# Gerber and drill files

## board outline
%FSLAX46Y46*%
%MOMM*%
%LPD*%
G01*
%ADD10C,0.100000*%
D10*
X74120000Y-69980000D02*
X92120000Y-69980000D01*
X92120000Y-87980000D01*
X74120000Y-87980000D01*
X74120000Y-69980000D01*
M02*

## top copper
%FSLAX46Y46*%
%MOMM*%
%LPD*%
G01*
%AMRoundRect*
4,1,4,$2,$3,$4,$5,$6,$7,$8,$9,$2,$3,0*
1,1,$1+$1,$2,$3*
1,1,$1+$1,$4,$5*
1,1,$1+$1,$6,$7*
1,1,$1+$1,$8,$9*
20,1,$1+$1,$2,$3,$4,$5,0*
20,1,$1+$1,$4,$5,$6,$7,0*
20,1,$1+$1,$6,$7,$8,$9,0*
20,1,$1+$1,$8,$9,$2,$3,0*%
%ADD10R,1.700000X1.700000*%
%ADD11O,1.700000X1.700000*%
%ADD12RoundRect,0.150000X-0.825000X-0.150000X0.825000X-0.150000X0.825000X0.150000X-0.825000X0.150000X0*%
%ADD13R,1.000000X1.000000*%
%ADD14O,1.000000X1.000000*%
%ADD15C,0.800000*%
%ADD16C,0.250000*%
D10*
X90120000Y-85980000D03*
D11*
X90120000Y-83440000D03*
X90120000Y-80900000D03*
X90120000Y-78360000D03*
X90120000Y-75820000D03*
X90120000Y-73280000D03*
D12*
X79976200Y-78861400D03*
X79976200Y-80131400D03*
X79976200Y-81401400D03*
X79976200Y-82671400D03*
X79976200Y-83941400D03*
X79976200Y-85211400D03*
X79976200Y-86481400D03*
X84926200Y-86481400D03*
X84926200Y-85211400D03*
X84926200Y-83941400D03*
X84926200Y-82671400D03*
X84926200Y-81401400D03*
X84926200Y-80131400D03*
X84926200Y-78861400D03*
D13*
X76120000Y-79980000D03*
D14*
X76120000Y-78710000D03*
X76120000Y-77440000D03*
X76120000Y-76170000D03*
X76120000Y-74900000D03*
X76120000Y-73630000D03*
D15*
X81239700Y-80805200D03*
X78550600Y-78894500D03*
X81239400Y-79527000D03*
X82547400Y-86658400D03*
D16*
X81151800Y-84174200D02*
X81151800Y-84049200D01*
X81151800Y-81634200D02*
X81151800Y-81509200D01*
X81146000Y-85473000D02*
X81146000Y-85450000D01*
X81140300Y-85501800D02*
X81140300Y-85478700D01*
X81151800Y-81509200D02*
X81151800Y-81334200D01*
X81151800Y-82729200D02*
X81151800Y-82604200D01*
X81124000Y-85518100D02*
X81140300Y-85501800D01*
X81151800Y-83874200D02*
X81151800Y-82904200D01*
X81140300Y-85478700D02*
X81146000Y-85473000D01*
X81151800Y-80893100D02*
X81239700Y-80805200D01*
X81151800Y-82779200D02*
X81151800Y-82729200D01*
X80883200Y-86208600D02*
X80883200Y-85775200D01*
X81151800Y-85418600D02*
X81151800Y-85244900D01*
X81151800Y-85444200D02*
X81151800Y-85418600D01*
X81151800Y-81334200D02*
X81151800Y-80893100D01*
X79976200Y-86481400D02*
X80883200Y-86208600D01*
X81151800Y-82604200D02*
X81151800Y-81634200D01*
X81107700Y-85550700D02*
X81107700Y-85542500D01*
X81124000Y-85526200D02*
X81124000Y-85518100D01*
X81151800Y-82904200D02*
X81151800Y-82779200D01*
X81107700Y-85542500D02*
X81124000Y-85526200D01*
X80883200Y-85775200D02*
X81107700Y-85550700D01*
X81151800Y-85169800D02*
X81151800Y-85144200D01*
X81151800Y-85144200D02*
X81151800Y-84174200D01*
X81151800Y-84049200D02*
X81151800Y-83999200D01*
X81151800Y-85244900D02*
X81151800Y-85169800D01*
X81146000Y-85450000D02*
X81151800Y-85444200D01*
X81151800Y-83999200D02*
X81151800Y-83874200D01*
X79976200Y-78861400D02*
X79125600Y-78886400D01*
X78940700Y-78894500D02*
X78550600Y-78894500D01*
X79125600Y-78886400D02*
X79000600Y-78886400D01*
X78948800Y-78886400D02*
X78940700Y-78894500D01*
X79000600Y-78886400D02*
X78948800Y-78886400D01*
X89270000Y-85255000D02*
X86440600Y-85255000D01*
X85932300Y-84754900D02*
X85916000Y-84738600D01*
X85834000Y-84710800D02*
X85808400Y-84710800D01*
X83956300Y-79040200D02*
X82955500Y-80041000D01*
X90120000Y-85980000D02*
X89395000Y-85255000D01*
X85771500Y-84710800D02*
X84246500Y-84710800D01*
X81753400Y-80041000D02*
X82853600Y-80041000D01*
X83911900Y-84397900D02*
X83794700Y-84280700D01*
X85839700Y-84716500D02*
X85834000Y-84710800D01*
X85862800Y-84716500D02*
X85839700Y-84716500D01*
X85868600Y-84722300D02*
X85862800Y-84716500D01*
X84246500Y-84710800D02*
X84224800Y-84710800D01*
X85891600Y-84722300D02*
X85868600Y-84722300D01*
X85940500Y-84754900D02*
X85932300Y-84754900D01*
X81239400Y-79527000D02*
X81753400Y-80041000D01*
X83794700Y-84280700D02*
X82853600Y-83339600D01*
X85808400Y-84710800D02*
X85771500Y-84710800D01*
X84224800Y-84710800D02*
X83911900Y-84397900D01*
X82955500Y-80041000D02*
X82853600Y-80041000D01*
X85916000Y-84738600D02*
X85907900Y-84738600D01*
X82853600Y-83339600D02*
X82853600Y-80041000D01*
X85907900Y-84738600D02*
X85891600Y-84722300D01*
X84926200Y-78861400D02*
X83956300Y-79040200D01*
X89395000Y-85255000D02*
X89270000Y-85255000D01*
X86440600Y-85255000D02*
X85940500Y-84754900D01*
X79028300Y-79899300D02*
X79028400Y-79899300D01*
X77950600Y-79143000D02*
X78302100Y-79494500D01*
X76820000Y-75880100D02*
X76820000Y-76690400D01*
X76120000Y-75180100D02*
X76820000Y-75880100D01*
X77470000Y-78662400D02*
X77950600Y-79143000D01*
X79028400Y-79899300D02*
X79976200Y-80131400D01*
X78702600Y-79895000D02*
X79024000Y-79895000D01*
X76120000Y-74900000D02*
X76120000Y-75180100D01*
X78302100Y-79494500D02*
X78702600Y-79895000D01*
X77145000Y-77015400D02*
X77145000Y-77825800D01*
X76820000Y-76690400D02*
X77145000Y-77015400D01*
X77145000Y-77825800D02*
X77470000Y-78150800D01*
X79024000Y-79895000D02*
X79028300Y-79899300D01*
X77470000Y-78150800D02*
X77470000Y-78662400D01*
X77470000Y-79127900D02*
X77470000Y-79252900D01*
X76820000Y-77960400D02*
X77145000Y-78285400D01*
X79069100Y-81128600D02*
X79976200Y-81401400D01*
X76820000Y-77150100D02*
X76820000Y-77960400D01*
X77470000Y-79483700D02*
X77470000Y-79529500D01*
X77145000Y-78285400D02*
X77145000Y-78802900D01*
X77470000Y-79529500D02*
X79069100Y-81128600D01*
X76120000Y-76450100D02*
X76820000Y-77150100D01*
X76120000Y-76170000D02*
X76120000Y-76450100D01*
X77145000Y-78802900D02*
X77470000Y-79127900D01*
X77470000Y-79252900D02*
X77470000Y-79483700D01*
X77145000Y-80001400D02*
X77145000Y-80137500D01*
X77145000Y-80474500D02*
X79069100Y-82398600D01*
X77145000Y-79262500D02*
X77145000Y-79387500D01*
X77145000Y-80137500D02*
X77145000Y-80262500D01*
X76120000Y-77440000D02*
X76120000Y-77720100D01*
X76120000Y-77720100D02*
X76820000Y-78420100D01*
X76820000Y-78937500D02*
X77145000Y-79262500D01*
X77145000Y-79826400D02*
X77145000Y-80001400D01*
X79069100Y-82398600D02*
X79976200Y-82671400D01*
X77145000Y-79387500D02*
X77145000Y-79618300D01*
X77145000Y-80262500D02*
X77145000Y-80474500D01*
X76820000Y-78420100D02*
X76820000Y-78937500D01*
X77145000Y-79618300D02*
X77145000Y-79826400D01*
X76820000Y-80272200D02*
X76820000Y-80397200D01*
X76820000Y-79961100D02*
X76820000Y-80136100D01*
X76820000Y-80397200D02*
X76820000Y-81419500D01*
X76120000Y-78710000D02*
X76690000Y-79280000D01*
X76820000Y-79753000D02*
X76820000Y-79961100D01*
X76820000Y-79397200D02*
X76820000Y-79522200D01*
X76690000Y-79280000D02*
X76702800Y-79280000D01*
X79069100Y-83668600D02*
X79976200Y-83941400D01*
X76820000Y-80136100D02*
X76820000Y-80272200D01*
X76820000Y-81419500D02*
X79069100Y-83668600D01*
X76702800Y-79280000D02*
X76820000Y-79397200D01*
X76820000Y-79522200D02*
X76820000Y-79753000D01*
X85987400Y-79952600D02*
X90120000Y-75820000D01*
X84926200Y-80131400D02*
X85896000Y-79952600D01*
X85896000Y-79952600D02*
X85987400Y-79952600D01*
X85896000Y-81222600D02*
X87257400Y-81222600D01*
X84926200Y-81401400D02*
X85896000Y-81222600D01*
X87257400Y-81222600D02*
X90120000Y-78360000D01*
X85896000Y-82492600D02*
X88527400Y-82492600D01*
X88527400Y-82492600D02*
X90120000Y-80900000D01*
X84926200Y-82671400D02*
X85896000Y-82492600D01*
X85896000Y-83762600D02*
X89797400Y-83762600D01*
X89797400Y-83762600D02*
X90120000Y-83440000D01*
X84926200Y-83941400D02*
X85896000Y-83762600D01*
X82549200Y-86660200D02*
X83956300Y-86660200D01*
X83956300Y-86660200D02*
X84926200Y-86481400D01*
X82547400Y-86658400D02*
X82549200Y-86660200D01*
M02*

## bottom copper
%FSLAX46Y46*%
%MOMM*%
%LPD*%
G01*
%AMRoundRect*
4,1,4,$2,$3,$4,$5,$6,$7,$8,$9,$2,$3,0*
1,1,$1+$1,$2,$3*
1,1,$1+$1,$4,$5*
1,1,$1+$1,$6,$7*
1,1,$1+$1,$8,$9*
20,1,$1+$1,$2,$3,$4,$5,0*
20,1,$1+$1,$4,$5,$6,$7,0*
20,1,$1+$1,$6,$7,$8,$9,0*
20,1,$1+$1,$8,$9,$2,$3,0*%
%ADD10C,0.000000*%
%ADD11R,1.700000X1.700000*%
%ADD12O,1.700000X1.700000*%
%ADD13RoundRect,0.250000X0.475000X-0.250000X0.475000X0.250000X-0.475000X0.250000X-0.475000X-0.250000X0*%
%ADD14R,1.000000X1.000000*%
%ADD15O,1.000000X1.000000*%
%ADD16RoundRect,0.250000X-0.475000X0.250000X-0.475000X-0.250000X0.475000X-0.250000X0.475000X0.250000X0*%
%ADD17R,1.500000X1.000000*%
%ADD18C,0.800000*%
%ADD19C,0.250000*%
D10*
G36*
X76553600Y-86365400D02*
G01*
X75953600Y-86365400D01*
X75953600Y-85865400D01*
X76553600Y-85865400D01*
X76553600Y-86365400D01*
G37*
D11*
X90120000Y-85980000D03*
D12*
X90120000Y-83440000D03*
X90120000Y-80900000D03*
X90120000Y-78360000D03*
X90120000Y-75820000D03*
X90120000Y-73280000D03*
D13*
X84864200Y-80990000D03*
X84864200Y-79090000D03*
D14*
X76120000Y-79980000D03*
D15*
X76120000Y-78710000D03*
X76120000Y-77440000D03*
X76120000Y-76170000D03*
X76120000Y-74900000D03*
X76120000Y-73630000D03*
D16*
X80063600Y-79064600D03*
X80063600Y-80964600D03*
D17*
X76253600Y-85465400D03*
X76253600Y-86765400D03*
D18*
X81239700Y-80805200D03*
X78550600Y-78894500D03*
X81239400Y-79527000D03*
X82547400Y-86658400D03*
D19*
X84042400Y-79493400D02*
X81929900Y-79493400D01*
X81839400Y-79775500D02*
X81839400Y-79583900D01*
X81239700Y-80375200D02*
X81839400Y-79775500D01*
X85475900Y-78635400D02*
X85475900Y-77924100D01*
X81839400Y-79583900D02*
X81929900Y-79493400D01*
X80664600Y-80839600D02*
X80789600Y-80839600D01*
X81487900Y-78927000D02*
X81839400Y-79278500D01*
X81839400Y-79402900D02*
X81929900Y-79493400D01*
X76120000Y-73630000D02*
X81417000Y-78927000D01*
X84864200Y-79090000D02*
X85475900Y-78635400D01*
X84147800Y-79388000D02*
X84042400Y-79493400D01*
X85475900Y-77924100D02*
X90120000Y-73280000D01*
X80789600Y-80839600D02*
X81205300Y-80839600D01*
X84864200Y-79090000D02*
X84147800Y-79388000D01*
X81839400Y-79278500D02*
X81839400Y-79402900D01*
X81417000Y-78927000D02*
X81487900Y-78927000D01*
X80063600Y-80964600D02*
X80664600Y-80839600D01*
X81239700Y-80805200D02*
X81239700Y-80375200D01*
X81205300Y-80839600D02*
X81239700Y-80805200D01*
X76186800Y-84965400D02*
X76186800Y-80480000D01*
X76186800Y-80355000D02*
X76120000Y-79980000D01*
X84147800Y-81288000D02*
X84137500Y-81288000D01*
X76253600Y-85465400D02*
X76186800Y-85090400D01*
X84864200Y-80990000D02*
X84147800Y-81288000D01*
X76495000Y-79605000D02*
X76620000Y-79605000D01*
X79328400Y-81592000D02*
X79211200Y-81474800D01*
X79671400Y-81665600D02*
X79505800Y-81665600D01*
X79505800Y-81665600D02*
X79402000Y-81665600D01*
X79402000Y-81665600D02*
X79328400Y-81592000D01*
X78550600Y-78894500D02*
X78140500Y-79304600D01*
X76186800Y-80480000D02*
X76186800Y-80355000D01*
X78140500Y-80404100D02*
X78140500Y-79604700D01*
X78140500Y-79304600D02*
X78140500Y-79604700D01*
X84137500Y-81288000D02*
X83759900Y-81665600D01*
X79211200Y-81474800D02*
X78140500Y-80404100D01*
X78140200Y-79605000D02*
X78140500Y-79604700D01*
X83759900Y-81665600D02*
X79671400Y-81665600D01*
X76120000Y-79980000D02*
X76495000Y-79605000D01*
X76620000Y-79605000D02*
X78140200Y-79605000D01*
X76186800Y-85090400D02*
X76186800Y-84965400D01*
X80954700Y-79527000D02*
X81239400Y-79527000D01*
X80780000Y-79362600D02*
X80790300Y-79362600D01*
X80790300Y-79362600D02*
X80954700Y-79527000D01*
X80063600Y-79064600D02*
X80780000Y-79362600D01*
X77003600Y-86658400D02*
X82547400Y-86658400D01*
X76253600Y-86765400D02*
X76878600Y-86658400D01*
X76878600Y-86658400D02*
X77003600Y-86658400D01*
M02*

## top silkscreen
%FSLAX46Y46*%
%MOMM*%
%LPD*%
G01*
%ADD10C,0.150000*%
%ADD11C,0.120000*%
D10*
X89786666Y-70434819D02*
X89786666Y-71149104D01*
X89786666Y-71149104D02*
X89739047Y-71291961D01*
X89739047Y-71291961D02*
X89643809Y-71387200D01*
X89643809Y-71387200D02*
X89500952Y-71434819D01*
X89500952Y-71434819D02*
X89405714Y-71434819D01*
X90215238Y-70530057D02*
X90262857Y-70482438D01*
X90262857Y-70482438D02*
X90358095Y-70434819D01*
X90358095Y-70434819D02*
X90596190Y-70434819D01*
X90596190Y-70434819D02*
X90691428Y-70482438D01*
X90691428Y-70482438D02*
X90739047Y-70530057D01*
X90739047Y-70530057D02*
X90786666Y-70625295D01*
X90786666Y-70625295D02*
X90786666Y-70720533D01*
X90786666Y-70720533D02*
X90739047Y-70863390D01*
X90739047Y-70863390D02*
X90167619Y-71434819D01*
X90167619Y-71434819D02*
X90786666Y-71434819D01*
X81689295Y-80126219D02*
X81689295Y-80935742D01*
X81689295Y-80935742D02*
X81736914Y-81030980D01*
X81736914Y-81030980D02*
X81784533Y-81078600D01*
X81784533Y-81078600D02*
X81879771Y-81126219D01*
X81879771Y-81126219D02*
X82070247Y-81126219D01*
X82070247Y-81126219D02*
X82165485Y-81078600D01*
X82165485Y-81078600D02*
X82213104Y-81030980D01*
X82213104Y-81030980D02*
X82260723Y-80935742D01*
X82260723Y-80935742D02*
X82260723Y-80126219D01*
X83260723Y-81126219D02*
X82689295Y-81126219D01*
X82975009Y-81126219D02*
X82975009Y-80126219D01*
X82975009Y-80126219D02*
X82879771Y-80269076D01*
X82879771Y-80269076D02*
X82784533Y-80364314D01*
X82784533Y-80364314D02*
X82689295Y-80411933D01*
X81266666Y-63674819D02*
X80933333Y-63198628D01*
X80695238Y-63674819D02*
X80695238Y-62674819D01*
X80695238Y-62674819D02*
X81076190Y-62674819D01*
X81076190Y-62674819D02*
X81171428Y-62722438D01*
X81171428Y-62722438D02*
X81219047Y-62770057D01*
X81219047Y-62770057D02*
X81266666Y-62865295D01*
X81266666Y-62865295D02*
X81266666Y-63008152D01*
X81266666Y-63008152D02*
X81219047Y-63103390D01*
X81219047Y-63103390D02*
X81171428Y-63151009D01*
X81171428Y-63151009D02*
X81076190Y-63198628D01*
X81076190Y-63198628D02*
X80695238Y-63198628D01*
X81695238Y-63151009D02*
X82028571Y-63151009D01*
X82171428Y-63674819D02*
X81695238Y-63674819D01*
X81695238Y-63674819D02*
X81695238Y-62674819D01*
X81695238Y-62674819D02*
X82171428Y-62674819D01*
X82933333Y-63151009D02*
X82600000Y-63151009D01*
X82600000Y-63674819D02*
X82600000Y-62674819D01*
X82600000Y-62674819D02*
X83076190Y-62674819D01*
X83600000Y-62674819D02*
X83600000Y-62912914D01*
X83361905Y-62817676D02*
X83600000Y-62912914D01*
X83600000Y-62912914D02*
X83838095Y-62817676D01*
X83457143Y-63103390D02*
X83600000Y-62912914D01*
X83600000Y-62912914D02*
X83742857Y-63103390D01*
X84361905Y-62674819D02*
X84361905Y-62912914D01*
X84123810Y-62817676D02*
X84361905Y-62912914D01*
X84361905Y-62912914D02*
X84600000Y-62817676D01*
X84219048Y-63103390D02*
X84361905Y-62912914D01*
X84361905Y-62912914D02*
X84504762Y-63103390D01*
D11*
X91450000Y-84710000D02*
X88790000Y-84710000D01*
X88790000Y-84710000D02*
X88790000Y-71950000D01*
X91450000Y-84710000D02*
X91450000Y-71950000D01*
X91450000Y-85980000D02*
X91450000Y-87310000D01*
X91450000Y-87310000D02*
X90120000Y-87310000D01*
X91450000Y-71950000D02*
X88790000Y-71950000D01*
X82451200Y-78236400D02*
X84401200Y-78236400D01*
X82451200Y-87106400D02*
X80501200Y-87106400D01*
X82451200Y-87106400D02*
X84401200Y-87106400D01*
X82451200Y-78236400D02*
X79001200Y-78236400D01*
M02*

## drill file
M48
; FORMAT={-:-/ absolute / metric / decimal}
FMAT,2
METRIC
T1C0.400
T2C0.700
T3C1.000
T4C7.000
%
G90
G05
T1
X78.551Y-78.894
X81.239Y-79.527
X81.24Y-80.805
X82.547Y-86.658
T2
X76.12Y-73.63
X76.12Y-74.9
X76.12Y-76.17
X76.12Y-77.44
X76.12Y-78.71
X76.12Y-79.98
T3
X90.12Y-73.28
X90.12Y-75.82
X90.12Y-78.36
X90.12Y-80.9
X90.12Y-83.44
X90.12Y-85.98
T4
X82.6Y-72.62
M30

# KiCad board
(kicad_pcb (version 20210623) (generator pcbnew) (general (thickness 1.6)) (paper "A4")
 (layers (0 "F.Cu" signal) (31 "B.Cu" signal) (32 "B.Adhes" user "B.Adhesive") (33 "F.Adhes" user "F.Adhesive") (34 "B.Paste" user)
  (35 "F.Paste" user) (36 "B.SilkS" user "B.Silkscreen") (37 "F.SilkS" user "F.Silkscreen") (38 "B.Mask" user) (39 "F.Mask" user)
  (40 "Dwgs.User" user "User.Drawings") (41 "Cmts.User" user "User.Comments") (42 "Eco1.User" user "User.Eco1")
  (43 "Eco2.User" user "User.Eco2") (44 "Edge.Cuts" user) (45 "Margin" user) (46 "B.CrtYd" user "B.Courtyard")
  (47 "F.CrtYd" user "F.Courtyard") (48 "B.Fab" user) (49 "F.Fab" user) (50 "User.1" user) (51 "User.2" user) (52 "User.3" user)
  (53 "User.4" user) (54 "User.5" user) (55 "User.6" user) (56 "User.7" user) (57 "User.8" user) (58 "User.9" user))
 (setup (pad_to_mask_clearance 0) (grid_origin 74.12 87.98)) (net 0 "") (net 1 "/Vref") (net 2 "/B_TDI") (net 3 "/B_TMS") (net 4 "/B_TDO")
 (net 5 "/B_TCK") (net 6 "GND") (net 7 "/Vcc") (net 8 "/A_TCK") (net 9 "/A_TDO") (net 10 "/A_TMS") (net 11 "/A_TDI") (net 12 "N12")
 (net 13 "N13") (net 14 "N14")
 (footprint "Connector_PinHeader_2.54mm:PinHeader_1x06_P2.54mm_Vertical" (layer "F.Cu") (at 90.12 85.98 180)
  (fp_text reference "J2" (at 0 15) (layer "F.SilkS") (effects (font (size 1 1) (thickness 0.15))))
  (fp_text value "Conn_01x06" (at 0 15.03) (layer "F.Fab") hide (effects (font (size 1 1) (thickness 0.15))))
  (fp_line (start -1.33 1.27) (end 1.33 1.27) (layer "F.SilkS") (width 0.12))
  (fp_line (start 1.33 1.27) (end 1.33 14.03) (layer "F.SilkS") (width 0.12))
  (fp_line (start -1.33 1.27) (end -1.33 14.03) (layer "F.SilkS") (width 0.12))
  (fp_line (start -1.33 0) (end -1.33 -1.33) (layer "F.SilkS") (width 0.12))
  (fp_line (start -1.33 -1.33) (end 0 -1.33) (layer "F.SilkS") (width 0.12))
  (fp_line (start -1.33 14.03) (end 1.33 14.03) (layer "F.SilkS") (width 0.12))
  (pad "1" thru_hole rect locked (at 0 0 180) (size 1.7 1.7) (drill 1) (layers *.Cu *.Mask) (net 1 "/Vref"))
  (pad "2" thru_hole oval locked (at 0 2.54 180) (size 1.7 1.7) (drill 1) (layers *.Cu *.Mask) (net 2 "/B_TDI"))
  (pad "3" thru_hole oval locked (at 0 5.08 180) (size 1.7 1.7) (drill 1) (layers *.Cu *.Mask) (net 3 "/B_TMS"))
  (pad "4" thru_hole oval locked (at 0 7.62 180) (size 1.7 1.7) (drill 1) (layers *.Cu *.Mask) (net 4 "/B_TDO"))
  (pad "5" thru_hole oval locked (at 0 10.16 180) (size 1.7 1.7) (drill 1) (layers *.Cu *.Mask) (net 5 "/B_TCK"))
  (pad "6" thru_hole oval locked (at 0 12.7 180) (size 1.7 1.7) (drill 1) (layers *.Cu *.Mask) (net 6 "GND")))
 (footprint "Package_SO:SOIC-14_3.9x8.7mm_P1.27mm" (layer "F.Cu") (at 82.4512 82.6714)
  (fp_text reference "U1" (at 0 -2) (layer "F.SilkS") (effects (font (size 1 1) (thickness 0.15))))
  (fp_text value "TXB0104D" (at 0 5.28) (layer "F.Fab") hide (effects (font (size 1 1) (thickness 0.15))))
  (fp_line (start 0 -4.435) (end 1.95 -4.435) (layer "F.SilkS") (width 0.12))
  (fp_line (start 0 4.435) (end -1.95 4.435) (layer "F.SilkS") (width 0.12))
  (fp_line (start 0 4.435) (end 1.95 4.435) (layer "F.SilkS") (width 0.12))
  (fp_line (start 0 -4.435) (end -3.45 -4.435) (layer "F.SilkS") (width 0.12))
  (pad "1" smd roundrect locked (at -2.475 -3.81) (size 1.95 0.6) (layers "F.Cu" "F.Paste" "F.Mask") (roundrect_rratio 0.25) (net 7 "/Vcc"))
  (pad "2" smd roundrect locked (at -2.475 -2.54) (size 1.95 0.6) (layers "F.Cu" "F.Paste" "F.Mask") (roundrect_rratio 0.25)
   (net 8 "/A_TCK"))
  (pad "3" smd roundrect locked (at -2.475 -1.27) (size 1.95 0.6) (layers "F.Cu" "F.Paste" "F.Mask") (roundrect_rratio 0.25)
   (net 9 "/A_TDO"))
  (pad "4" smd roundrect locked (at -2.475 0) (size 1.95 0.6) (layers "F.Cu" "F.Paste" "F.Mask") (roundrect_rratio 0.25) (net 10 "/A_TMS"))
  (pad "5" smd roundrect locked (at -2.475 1.27) (size 1.95 0.6) (layers "F.Cu" "F.Paste" "F.Mask") (roundrect_rratio 0.25)
   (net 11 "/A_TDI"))
  (pad "6" smd roundrect locked (at -2.475 2.54) (size 1.95 0.6) (layers "F.Cu" "F.Paste" "F.Mask") (roundrect_rratio 0.25) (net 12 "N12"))
  (pad "7" smd roundrect locked (at -2.475 3.81) (size 1.95 0.6) (layers "F.Cu" "F.Paste" "F.Mask") (roundrect_rratio 0.25) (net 6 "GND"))
  (pad "8" smd roundrect locked (at 2.475 3.81) (size 1.95 0.6) (layers "F.Cu" "F.Paste" "F.Mask") (roundrect_rratio 0.25) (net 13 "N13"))
  (pad "9" smd roundrect locked (at 2.475 2.54) (size 1.95 0.6) (layers "F.Cu" "F.Paste" "F.Mask") (roundrect_rratio 0.25) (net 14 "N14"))
  (pad "10" smd roundrect locked (at 2.475 1.27) (size 1.95 0.6) (layers "F.Cu" "F.Paste" "F.Mask") (roundrect_rratio 0.25) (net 2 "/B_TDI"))
  (pad "11" smd roundrect locked (at 2.475 0) (size 1.95 0.6) (layers "F.Cu" "F.Paste" "F.Mask") (roundrect_rratio 0.25) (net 3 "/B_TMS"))
  (pad "12" smd roundrect locked (at 2.475 -1.27) (size 1.95 0.6) (layers "F.Cu" "F.Paste" "F.Mask") (roundrect_rratio 0.25)
   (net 4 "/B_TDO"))
  (pad "13" smd roundrect locked (at 2.475 -2.54) (size 1.95 0.6) (layers "F.Cu" "F.Paste" "F.Mask") (roundrect_rratio 0.25)
   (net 5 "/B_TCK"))
  (pad "14" smd roundrect locked (at 2.475 -3.81) (size 1.95 0.6) (layers "F.Cu" "F.Paste" "F.Mask") (roundrect_rratio 0.25) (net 1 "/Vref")))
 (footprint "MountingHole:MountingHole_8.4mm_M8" (layer "F.Cu") (at 82.6 72.62)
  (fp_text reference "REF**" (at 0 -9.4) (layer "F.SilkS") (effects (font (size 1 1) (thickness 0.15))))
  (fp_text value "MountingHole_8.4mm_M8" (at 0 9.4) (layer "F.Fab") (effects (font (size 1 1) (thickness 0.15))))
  (pad "" np_thru_hole circle (at 0 0) (size 7 7) (drill 7) (layers F&B.Cu *.Mask)))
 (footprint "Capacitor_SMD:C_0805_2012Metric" (layer "B.Cu") (at 84.8642 80.04 90)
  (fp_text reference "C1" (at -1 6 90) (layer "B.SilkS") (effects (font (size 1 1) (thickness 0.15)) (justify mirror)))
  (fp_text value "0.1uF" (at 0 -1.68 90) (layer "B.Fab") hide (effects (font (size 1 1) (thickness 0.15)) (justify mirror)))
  (pad "1" smd roundrect locked (at -0.95 0 90) (size 1 1.45) (layers "B.Cu" "B.Paste" "B.Mask") (roundrect_rratio 0.25) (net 7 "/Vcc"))
  (pad "2" smd roundrect locked (at 0.95 0 90) (size 1 1.45) (layers "B.Cu" "B.Paste" "B.Mask") (roundrect_rratio 0.25) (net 6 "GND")))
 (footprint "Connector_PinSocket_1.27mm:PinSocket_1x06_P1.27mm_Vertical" (layer "B.Cu") (at 76.12 79.98)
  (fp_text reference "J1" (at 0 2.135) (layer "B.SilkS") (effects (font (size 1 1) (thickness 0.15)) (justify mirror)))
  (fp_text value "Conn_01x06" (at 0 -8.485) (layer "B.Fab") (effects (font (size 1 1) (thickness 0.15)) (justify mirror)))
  (pad "1" thru_hole rect locked (at 0 0) (size 1 1) (drill 0.7) (layers *.Cu *.Mask) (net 7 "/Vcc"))
  (pad "2" thru_hole oval locked (at 0 -1.27) (size 1 1) (drill 0.7) (layers *.Cu *.Mask) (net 11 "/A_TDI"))
  (pad "3" thru_hole oval locked (at 0 -2.54) (size 1 1) (drill 0.7) (layers *.Cu *.Mask) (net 10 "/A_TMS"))
  (pad "4" thru_hole oval locked (at 0 -3.81) (size 1 1) (drill 0.7) (layers *.Cu *.Mask) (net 9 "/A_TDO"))
  (pad "5" thru_hole oval locked (at 0 -5.08) (size 1 1) (drill 0.7) (layers *.Cu *.Mask) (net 8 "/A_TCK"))
  (pad "6" thru_hole oval locked (at 0 -6.35) (size 1 1) (drill 0.7) (layers *.Cu *.Mask) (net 6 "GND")))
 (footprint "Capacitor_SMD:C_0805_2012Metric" (layer "B.Cu") (at 80.0636 80.0146 -90)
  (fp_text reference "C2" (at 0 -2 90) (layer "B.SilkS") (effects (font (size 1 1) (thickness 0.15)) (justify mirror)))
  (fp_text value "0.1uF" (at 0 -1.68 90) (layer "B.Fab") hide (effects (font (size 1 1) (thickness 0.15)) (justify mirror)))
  (pad "1" smd roundrect locked (at -0.95 0 270) (size 1 1.45) (layers "B.Cu" "B.Paste" "B.Mask") (roundrect_rratio 0.25) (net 1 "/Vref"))
  (pad "2" smd roundrect locked (at 0.95 0 270) (size 1 1.45) (layers "B.Cu" "B.Paste" "B.Mask") (roundrect_rratio 0.25) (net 6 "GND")))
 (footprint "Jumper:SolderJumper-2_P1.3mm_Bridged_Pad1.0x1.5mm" (layer "B.Cu") (at 76.2536 86.1154 -90)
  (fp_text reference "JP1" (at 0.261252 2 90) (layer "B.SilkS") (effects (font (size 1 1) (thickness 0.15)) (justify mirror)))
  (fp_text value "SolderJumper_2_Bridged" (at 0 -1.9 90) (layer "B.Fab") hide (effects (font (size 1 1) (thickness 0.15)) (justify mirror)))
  (fp_poly (pts (xy -0.25 0.3) (xy 0.25 0.3) (xy 0.25 -0.3) (xy -0.25 -0.3)) (layer "B.Cu") (width 0) (fill solid))
  (pad "1" smd rect locked (at -0.65 0 270) (size 1 1.5) (layers "B.Cu" "B.Mask") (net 7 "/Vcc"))
  (pad "2" smd rect locked (at 0.65 0 270) (size 1 1.5) (layers "B.Cu" "B.Mask") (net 13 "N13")))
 (gr_rect (start 92.12 87.98) (end 74.12 69.98) (layer "Edge.Cuts") (width 0.1) (fill none))
 (segment (start 81.1518 84.1742) (end 81.1518 84.0492) (width 0.25) (layer "F.Cu") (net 6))
 (segment (start 81.1518 81.6342) (end 81.1518 81.5092) (width 0.25) (layer "F.Cu") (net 6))
 (segment (start 81.146 85.473) (end 81.146 85.45) (width 0.25) (layer "F.Cu") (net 6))
 (segment (start 81.1403 85.5018) (end 81.1403 85.4787) (width 0.25) (layer "F.Cu") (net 6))
 (segment (start 81.1518 81.5092) (end 81.1518 81.3342) (width 0.25) (layer "F.Cu") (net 6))
 (segment (start 81.1518 82.7292) (end 81.1518 82.6042) (width 0.25) (layer "F.Cu") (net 6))
 (segment (start 81.124 85.5181) (end 81.1403 85.5018) (width 0.25) (layer "F.Cu") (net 6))
 (segment (start 81.1518 83.8742) (end 81.1518 82.9042) (width 0.25) (layer "F.Cu") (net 6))
 (segment (start 81.1403 85.4787) (end 81.146 85.473) (width 0.25) (layer "F.Cu") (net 6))
 (segment (start 81.1518 80.8931) (end 81.2397 80.8052) (width 0.25) (layer "F.Cu") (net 6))
 (segment (start 81.1518 82.7792) (end 81.1518 82.7292) (width 0.25) (layer "F.Cu") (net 6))
 (segment (start 80.8832 86.2086) (end 80.8832 85.7752) (width 0.25) (layer "F.Cu") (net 6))
 (segment (start 81.1518 85.4186) (end 81.1518 85.2449) (width 0.25) (layer "F.Cu") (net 6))
 (segment (start 81.1518 85.4442) (end 81.1518 85.4186) (width 0.25) (layer "F.Cu") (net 6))
 (segment (start 81.1518 81.3342) (end 81.1518 80.8931) (width 0.25) (layer "F.Cu") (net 6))
 (segment (start 79.9762 86.4814) (end 80.8832 86.2086) (width 0.25) (layer "F.Cu") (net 6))
 (segment (start 81.1518 82.6042) (end 81.1518 81.6342) (width 0.25) (layer "F.Cu") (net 6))
 (segment (start 81.1077 85.5507) (end 81.1077 85.5425) (width 0.25) (layer "F.Cu") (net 6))
 (segment (start 81.124 85.5262) (end 81.124 85.5181) (width 0.25) (layer "F.Cu") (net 6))
 (segment (start 81.1518 82.9042) (end 81.1518 82.7792) (width 0.25) (layer "F.Cu") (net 6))
 (segment (start 81.1077 85.5425) (end 81.124 85.5262) (width 0.25) (layer "F.Cu") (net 6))
 (segment (start 80.8832 85.7752) (end 81.1077 85.5507) (width 0.25) (layer "F.Cu") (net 6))
 (segment (start 81.1518 85.1698) (end 81.1518 85.1442) (width 0.25) (layer "F.Cu") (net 6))
 (segment (start 81.1518 85.1442) (end 81.1518 84.1742) (width 0.25) (layer "F.Cu") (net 6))
 (segment (start 81.1518 84.0492) (end 81.1518 83.9992) (width 0.25) (layer "F.Cu") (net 6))
 (segment (start 81.1518 85.2449) (end 81.1518 85.1698) (width 0.25) (layer "F.Cu") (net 6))
 (segment (start 81.146 85.45) (end 81.1518 85.4442) (width 0.25) (layer "F.Cu") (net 6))
 (segment (start 81.1518 83.9992) (end 81.1518 83.8742) (width 0.25) (layer "F.Cu") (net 6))
 (via (at 81.2397 80.8052) (size 0.8) (drill 0.4) (layers "F.Cu" "B.Cu") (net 6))
 (segment (start 84.0424 79.4934) (end 81.9299 79.4934) (width 0.25) (layer "B.Cu") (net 6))
 (segment (start 81.8394 79.7755) (end 81.8394 79.5839) (width 0.25) (layer "B.Cu") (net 6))
 (segment (start 81.2397 80.3752) (end 81.8394 79.7755) (width 0.25) (layer "B.Cu") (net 6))
 (segment (start 85.4759 78.6354) (end 85.4759 77.9241) (width 0.25) (layer "B.Cu") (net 6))
 (segment (start 81.8394 79.5839) (end 81.9299 79.4934) (width 0.25) (layer "B.Cu") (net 6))
 (segment (start 80.6646 80.8396) (end 80.7896 80.8396) (width 0.25) (layer "B.Cu") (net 6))
 (segment (start 81.4879 78.927) (end 81.8394 79.2785) (width 0.25) (layer "B.Cu") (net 6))
 (segment (start 81.8394 79.4029) (end 81.9299 79.4934) (width 0.25) (layer "B.Cu") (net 6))
 (segment (start 76.12 73.63) (end 81.417 78.927) (width 0.25) (layer "B.Cu") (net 6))
 (segment (start 84.8642 79.09) (end 85.4759 78.6354) (width 0.25) (layer "B.Cu") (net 6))
 (segment (start 84.1478 79.388) (end 84.0424 79.4934) (width 0.25) (layer "B.Cu") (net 6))
 (segment (start 85.4759 77.9241) (end 90.12 73.28) (width 0.25) (layer "B.Cu") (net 6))
 (segment (start 80.7896 80.8396) (end 81.2053 80.8396) (width 0.25) (layer "B.Cu") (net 6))
 (segment (start 84.8642 79.09) (end 84.1478 79.388) (width 0.25) (layer "B.Cu") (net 6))
 (segment (start 81.8394 79.2785) (end 81.8394 79.4029) (width 0.25) (layer "B.Cu") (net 6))
 (segment (start 81.417 78.927) (end 81.4879 78.927) (width 0.25) (layer "B.Cu") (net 6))
 (segment (start 80.0636 80.9646) (end 80.6646 80.8396) (width 0.25) (layer "B.Cu") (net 6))
 (segment (start 81.2397 80.8052) (end 81.2397 80.3752) (width 0.25) (layer "B.Cu") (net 6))
 (segment (start 81.2053 80.8396) (end 81.2397 80.8052) (width 0.25) (layer "B.Cu") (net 6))
 (segment (start 79.9762 78.8614) (end 79.1256 78.8864) (width 0.25) (layer "F.Cu") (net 7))
 (segment (start 78.9407 78.8945) (end 78.5506 78.8945) (width 0.25) (layer "F.Cu") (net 7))
 (segment (start 79.1256 78.8864) (end 79.0006 78.8864) (width 0.25) (layer "F.Cu") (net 7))
 (segment (start 78.9488 78.8864) (end 78.9407 78.8945) (width 0.25) (layer "F.Cu") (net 7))
 (segment (start 79.0006 78.8864) (end 78.9488 78.8864) (width 0.25) (layer "F.Cu") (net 7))
 (via (at 78.5506 78.8945) (size 0.8) (drill 0.4) (layers "F.Cu" "B.Cu") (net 7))
 (segment (start 76.1868 84.9654) (end 76.1868 80.48) (width 0.25) (layer "B.Cu") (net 7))
 (segment (start 76.1868 80.355) (end 76.12 79.98) (width 0.25) (layer "B.Cu") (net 7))
 (segment (start 84.1478 81.288) (end 84.1375 81.288) (width 0.25) (layer "B.Cu") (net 7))
 (segment (start 76.2536 85.4654) (end 76.1868 85.0904) (width 0.25) (layer "B.Cu") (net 7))
 (segment (start 84.8642 80.99) (end 84.1478 81.288) (width 0.25) (layer "B.Cu") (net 7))
 (segment (start 76.495 79.605) (end 76.62 79.605) (width 0.25) (layer "B.Cu") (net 7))
 (segment (start 79.3284 81.592) (end 79.2112 81.4748) (width 0.25) (layer "B.Cu") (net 7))
 (segment (start 79.6714 81.6656) (end 79.5058 81.6656) (width 0.25) (layer "B.Cu") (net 7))
 (segment (start 79.5058 81.6656) (end 79.402 81.6656) (width 0.25) (layer "B.Cu") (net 7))
 (segment (start 79.402 81.6656) (end 79.3284 81.592) (width 0.25) (layer "B.Cu") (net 7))
 (segment (start 78.5506 78.8945) (end 78.1405 79.3046) (width 0.25) (layer "B.Cu") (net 7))
 (segment (start 76.1868 80.48) (end 76.1868 80.355) (width 0.25) (layer "B.Cu") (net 7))
 (segment (start 78.1405 80.4041) (end 78.1405 79.6047) (width 0.25) (layer "B.Cu") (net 7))
 (segment (start 78.1405 79.3046) (end 78.1405 79.6047) (width 0.25) (layer "B.Cu") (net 7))
 (segment (start 84.1375 81.288) (end 83.7599 81.6656) (width 0.25) (layer "B.Cu") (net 7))
 (segment (start 79.2112 81.4748) (end 78.1405 80.4041) (width 0.25) (layer "B.Cu") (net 7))
 (segment (start 78.1402 79.605) (end 78.1405 79.6047) (width 0.25) (layer "B.Cu") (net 7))
 (segment (start 83.7599 81.6656) (end 79.6714 81.6656) (width 0.25) (layer "B.Cu") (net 7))
 (segment (start 76.12 79.98) (end 76.495 79.605) (width 0.25) (layer "B.Cu") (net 7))
 (segment (start 76.62 79.605) (end 78.1402 79.605) (width 0.25) (layer "B.Cu") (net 7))
 (segment (start 76.1868 85.0904) (end 76.1868 84.9654) (width 0.25) (layer "B.Cu") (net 7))
 (segment (start 89.27 85.255) (end 86.4406 85.255) (width 0.25) (layer "F.Cu") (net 1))
 (segment (start 85.9323 84.7549) (end 85.916 84.7386) (width 0.25) (layer "F.Cu") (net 1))
 (segment (start 85.834 84.7108) (end 85.8084 84.7108) (width 0.25) (layer "F.Cu") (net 1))
 (segment (start 83.9563 79.0402) (end 82.9555 80.041) (width 0.25) (layer "F.Cu") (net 1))
 (segment (start 90.12 85.98) (end 89.395 85.255) (width 0.25) (layer "F.Cu") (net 1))
 (segment (start 85.7715 84.7108) (end 84.2465 84.7108) (width 0.25) (layer "F.Cu") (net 1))
 (segment (start 81.7534 80.041) (end 82.8536 80.041) (width 0.25) (layer "F.Cu") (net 1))
 (segment (start 83.9119 84.3979) (end 83.7947 84.2807) (width 0.25) (layer "F.Cu") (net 1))
 (segment (start 85.8397 84.7165) (end 85.834 84.7108) (width 0.25) (layer "F.Cu") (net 1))
 (segment (start 85.8628 84.7165) (end 85.8397 84.7165) (width 0.25) (layer "F.Cu") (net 1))
 (segment (start 85.8686 84.7223) (end 85.8628 84.7165) (width 0.25) (layer "F.Cu") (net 1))
 (segment (start 84.2465 84.7108) (end 84.2248 84.7108) (width 0.25) (layer "F.Cu") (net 1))
 (segment (start 85.8916 84.7223) (end 85.8686 84.7223) (width 0.25) (layer "F.Cu") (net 1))
 (segment (start 85.9405 84.7549) (end 85.9323 84.7549) (width 0.25) (layer "F.Cu") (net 1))
 (segment (start 81.2394 79.527) (end 81.7534 80.041) (width 0.25) (layer "F.Cu") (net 1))
 (segment (start 83.7947 84.2807) (end 82.8536 83.3396) (width 0.25) (layer "F.Cu") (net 1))
 (segment (start 85.8084 84.7108) (end 85.7715 84.7108) (width 0.25) (layer "F.Cu") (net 1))
 (segment (start 84.2248 84.7108) (end 83.9119 84.3979) (width 0.25) (layer "F.Cu") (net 1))
 (segment (start 82.9555 80.041) (end 82.8536 80.041) (width 0.25) (layer "F.Cu") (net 1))
 (segment (start 85.916 84.7386) (end 85.9079 84.7386) (width 0.25) (layer "F.Cu") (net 1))
 (segment (start 82.8536 83.3396) (end 82.8536 80.041) (width 0.25) (layer "F.Cu") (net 1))
 (segment (start 85.9079 84.7386) (end 85.8916 84.7223) (width 0.25) (layer "F.Cu") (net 1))
 (segment (start 84.9262 78.8614) (end 83.9563 79.0402) (width 0.25) (layer "F.Cu") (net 1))
 (segment (start 89.395 85.255) (end 89.27 85.255) (width 0.25) (layer "F.Cu") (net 1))
 (segment (start 86.4406 85.255) (end 85.9405 84.7549) (width 0.25) (layer "F.Cu") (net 1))
 (via (at 81.2394 79.527) (size 0.8) (drill 0.4) (layers "F.Cu" "B.Cu") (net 1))
 (segment (start 80.9547 79.527) (end 81.2394 79.527) (width 0.25) (layer "B.Cu") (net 1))
 (segment (start 80.78 79.3626) (end 80.7903 79.3626) (width 0.25) (layer "B.Cu") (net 1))
 (segment (start 80.7903 79.3626) (end 80.9547 79.527) (width 0.25) (layer "B.Cu") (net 1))
 (segment (start 80.0636 79.0646) (end 80.78 79.3626) (width 0.25) (layer "B.Cu") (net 1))
 (segment (start 79.0283 79.8993) (end 79.0284 79.8993) (width 0.25) (layer "F.Cu") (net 8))
 (segment (start 77.9506 79.143) (end 78.3021 79.4945) (width 0.25) (layer "F.Cu") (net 8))
 (segment (start 76.82 75.8801) (end 76.82 76.6904) (width 0.25) (layer "F.Cu") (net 8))
 (segment (start 76.12 75.1801) (end 76.82 75.8801) (width 0.25) (layer "F.Cu") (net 8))
 (segment (start 77.47 78.6624) (end 77.9506 79.143) (width 0.25) (layer "F.Cu") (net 8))
 (segment (start 79.0284 79.8993) (end 79.9762 80.1314) (width 0.25) (layer "F.Cu") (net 8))
 (segment (start 78.7026 79.895) (end 79.024 79.895) (width 0.25) (layer "F.Cu") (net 8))
 (segment (start 76.12 74.9) (end 76.12 75.1801) (width 0.25) (layer "F.Cu") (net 8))
 (segment (start 78.3021 79.4945) (end 78.7026 79.895) (width 0.25) (layer "F.Cu") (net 8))
 (segment (start 77.145 77.0154) (end 77.145 77.8258) (width 0.25) (layer "F.Cu") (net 8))
 (segment (start 76.82 76.6904) (end 77.145 77.0154) (width 0.25) (layer "F.Cu") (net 8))
 (segment (start 77.145 77.8258) (end 77.47 78.1508) (width 0.25) (layer "F.Cu") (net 8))
 (segment (start 79.024 79.895) (end 79.0283 79.8993) (width 0.25) (layer "F.Cu") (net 8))
 (segment (start 77.47 78.1508) (end 77.47 78.6624) (width 0.25) (layer "F.Cu") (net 8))
 (segment (start 77.47 79.1279) (end 77.47 79.2529) (width 0.25) (layer "F.Cu") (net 9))
 (segment (start 76.82 77.9604) (end 77.145 78.2854) (width 0.25) (layer "F.Cu") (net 9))
 (segment (start 79.0691 81.1286) (end 79.9762 81.4014) (width 0.25) (layer "F.Cu") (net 9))
 (segment (start 76.82 77.1501) (end 76.82 77.9604) (width 0.25) (layer "F.Cu") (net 9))
 (segment (start 77.47 79.4837) (end 77.47 79.5295) (width 0.25) (layer "F.Cu") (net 9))
 (segment (start 77.145 78.2854) (end 77.145 78.8029) (width 0.25) (layer "F.Cu") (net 9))
 (segment (start 77.47 79.5295) (end 79.0691 81.1286) (width 0.25) (layer "F.Cu") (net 9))
 (segment (start 76.12 76.4501) (end 76.82 77.1501) (width 0.25) (layer "F.Cu") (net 9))
 (segment (start 76.12 76.17) (end 76.12 76.4501) (width 0.25) (layer "F.Cu") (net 9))
 (segment (start 77.145 78.8029) (end 77.47 79.1279) (width 0.25) (layer "F.Cu") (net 9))
 (segment (start 77.47 79.2529) (end 77.47 79.4837) (width 0.25) (layer "F.Cu") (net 9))
 (segment (start 77.145 80.0014) (end 77.145 80.1375) (width 0.25) (layer "F.Cu") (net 10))
 (segment (start 77.145 80.4745) (end 79.0691 82.3986) (width 0.25) (layer "F.Cu") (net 10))
 (segment (start 77.145 79.2625) (end 77.145 79.3875) (width 0.25) (layer "F.Cu") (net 10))
 (segment (start 77.145 80.1375) (end 77.145 80.2625) (width 0.25) (layer "F.Cu") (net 10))
 (segment (start 76.12 77.44) (end 76.12 77.7201) (width 0.25) (layer "F.Cu") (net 10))
 (segment (start 76.12 77.7201) (end 76.82 78.4201) (width 0.25) (layer "F.Cu") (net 10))
 (segment (start 76.82 78.9375) (end 77.145 79.2625) (width 0.25) (layer "F.Cu") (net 10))
 (segment (start 77.145 79.8264) (end 77.145 80.0014) (width 0.25) (layer "F.Cu") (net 10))
 (segment (start 79.0691 82.3986) (end 79.9762 82.6714) (width 0.25) (layer "F.Cu") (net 10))
 (segment (start 77.145 79.3875) (end 77.145 79.6183) (width 0.25) (layer "F.Cu") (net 10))
 (segment (start 77.145 80.2625) (end 77.145 80.4745) (width 0.25) (layer "F.Cu") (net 10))
 (segment (start 76.82 78.4201) (end 76.82 78.9375) (width 0.25) (layer "F.Cu") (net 10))
 (segment (start 77.145 79.6183) (end 77.145 79.8264) (width 0.25) (layer "F.Cu") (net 10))
 (segment (start 76.82 80.2722) (end 76.82 80.3972) (width 0.25) (layer "F.Cu") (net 11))
 (segment (start 76.82 79.9611) (end 76.82 80.1361) (width 0.25) (layer "F.Cu") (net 11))
 (segment (start 76.82 80.3972) (end 76.82 81.4195) (width 0.25) (layer "F.Cu") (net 11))
 (segment (start 76.12 78.71) (end 76.69 79.28) (width 0.25) (layer "F.Cu") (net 11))
 (segment (start 76.82 79.753) (end 76.82 79.9611) (width 0.25) (layer "F.Cu") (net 11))
 (segment (start 76.82 79.3972) (end 76.82 79.5222) (width 0.25) (layer "F.Cu") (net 11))
 (segment (start 76.69 79.28) (end 76.7028 79.28) (width 0.25) (layer "F.Cu") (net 11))
 (segment (start 79.0691 83.6686) (end 79.9762 83.9414) (width 0.25) (layer "F.Cu") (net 11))
 (segment (start 76.82 80.1361) (end 76.82 80.2722) (width 0.25) (layer "F.Cu") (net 11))
 (segment (start 76.82 81.4195) (end 79.0691 83.6686) (width 0.25) (layer "F.Cu") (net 11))
 (segment (start 76.7028 79.28) (end 76.82 79.3972) (width 0.25) (layer "F.Cu") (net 11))
 (segment (start 76.82 79.5222) (end 76.82 79.753) (width 0.25) (layer "F.Cu") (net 11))
 (segment (start 85.9874 79.9526) (end 90.12 75.82) (width 0.25) (layer "F.Cu") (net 5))
 (segment (start 84.9262 80.1314) (end 85.896 79.9526) (width 0.25) (layer "F.Cu") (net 5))
 (segment (start 85.896 79.9526) (end 85.9874 79.9526) (width 0.25) (layer "F.Cu") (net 5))
 (segment (start 85.896 81.2226) (end 87.2574 81.2226) (width 0.25) (layer "F.Cu") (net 4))
 (segment (start 84.9262 81.4014) (end 85.896 81.2226) (width 0.25) (layer "F.Cu") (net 4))
 (segment (start 87.2574 81.2226) (end 90.12 78.36) (width 0.25) (layer "F.Cu") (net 4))
 (segment (start 85.896 82.4926) (end 88.5274 82.4926) (width 0.25) (layer "F.Cu") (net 3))
 (segment (start 88.5274 82.4926) (end 90.12 80.9) (width 0.25) (layer "F.Cu") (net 3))
 (segment (start 84.9262 82.6714) (end 85.896 82.4926) (width 0.25) (layer "F.Cu") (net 3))
 (segment (start 85.896 83.7626) (end 89.7974 83.7626) (width 0.25) (layer "F.Cu") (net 2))
 (segment (start 89.7974 83.7626) (end 90.12 83.44) (width 0.25) (layer "F.Cu") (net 2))
 (segment (start 84.9262 83.9414) (end 85.896 83.7626) (width 0.25) (layer "F.Cu") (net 2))
 (segment (start 82.5492 86.6602) (end 83.9563 86.6602) (width 0.25) (layer "F.Cu") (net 13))
 (segment (start 83.9563 86.6602) (end 84.9262 86.4814) (width 0.25) (layer "F.Cu") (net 13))
 (segment (start 82.5474 86.6584) (end 82.5492 86.6602) (width 0.25) (layer "F.Cu") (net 13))
 (via (at 82.5474 86.6584) (size 0.8) (drill 0.4) (layers "F.Cu" "B.Cu") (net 13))
 (segment (start 77.0036 86.6584) (end 82.5474 86.6584) (width 0.25) (layer "B.Cu") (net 13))
 (segment (start 76.2536 86.7654) (end 76.8786 86.6584) (width 0.25) (layer "B.Cu") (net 13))
 (segment (start 76.8786 86.6584) (end 77.0036 86.6584) (width 0.25) (layer "B.Cu") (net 13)))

